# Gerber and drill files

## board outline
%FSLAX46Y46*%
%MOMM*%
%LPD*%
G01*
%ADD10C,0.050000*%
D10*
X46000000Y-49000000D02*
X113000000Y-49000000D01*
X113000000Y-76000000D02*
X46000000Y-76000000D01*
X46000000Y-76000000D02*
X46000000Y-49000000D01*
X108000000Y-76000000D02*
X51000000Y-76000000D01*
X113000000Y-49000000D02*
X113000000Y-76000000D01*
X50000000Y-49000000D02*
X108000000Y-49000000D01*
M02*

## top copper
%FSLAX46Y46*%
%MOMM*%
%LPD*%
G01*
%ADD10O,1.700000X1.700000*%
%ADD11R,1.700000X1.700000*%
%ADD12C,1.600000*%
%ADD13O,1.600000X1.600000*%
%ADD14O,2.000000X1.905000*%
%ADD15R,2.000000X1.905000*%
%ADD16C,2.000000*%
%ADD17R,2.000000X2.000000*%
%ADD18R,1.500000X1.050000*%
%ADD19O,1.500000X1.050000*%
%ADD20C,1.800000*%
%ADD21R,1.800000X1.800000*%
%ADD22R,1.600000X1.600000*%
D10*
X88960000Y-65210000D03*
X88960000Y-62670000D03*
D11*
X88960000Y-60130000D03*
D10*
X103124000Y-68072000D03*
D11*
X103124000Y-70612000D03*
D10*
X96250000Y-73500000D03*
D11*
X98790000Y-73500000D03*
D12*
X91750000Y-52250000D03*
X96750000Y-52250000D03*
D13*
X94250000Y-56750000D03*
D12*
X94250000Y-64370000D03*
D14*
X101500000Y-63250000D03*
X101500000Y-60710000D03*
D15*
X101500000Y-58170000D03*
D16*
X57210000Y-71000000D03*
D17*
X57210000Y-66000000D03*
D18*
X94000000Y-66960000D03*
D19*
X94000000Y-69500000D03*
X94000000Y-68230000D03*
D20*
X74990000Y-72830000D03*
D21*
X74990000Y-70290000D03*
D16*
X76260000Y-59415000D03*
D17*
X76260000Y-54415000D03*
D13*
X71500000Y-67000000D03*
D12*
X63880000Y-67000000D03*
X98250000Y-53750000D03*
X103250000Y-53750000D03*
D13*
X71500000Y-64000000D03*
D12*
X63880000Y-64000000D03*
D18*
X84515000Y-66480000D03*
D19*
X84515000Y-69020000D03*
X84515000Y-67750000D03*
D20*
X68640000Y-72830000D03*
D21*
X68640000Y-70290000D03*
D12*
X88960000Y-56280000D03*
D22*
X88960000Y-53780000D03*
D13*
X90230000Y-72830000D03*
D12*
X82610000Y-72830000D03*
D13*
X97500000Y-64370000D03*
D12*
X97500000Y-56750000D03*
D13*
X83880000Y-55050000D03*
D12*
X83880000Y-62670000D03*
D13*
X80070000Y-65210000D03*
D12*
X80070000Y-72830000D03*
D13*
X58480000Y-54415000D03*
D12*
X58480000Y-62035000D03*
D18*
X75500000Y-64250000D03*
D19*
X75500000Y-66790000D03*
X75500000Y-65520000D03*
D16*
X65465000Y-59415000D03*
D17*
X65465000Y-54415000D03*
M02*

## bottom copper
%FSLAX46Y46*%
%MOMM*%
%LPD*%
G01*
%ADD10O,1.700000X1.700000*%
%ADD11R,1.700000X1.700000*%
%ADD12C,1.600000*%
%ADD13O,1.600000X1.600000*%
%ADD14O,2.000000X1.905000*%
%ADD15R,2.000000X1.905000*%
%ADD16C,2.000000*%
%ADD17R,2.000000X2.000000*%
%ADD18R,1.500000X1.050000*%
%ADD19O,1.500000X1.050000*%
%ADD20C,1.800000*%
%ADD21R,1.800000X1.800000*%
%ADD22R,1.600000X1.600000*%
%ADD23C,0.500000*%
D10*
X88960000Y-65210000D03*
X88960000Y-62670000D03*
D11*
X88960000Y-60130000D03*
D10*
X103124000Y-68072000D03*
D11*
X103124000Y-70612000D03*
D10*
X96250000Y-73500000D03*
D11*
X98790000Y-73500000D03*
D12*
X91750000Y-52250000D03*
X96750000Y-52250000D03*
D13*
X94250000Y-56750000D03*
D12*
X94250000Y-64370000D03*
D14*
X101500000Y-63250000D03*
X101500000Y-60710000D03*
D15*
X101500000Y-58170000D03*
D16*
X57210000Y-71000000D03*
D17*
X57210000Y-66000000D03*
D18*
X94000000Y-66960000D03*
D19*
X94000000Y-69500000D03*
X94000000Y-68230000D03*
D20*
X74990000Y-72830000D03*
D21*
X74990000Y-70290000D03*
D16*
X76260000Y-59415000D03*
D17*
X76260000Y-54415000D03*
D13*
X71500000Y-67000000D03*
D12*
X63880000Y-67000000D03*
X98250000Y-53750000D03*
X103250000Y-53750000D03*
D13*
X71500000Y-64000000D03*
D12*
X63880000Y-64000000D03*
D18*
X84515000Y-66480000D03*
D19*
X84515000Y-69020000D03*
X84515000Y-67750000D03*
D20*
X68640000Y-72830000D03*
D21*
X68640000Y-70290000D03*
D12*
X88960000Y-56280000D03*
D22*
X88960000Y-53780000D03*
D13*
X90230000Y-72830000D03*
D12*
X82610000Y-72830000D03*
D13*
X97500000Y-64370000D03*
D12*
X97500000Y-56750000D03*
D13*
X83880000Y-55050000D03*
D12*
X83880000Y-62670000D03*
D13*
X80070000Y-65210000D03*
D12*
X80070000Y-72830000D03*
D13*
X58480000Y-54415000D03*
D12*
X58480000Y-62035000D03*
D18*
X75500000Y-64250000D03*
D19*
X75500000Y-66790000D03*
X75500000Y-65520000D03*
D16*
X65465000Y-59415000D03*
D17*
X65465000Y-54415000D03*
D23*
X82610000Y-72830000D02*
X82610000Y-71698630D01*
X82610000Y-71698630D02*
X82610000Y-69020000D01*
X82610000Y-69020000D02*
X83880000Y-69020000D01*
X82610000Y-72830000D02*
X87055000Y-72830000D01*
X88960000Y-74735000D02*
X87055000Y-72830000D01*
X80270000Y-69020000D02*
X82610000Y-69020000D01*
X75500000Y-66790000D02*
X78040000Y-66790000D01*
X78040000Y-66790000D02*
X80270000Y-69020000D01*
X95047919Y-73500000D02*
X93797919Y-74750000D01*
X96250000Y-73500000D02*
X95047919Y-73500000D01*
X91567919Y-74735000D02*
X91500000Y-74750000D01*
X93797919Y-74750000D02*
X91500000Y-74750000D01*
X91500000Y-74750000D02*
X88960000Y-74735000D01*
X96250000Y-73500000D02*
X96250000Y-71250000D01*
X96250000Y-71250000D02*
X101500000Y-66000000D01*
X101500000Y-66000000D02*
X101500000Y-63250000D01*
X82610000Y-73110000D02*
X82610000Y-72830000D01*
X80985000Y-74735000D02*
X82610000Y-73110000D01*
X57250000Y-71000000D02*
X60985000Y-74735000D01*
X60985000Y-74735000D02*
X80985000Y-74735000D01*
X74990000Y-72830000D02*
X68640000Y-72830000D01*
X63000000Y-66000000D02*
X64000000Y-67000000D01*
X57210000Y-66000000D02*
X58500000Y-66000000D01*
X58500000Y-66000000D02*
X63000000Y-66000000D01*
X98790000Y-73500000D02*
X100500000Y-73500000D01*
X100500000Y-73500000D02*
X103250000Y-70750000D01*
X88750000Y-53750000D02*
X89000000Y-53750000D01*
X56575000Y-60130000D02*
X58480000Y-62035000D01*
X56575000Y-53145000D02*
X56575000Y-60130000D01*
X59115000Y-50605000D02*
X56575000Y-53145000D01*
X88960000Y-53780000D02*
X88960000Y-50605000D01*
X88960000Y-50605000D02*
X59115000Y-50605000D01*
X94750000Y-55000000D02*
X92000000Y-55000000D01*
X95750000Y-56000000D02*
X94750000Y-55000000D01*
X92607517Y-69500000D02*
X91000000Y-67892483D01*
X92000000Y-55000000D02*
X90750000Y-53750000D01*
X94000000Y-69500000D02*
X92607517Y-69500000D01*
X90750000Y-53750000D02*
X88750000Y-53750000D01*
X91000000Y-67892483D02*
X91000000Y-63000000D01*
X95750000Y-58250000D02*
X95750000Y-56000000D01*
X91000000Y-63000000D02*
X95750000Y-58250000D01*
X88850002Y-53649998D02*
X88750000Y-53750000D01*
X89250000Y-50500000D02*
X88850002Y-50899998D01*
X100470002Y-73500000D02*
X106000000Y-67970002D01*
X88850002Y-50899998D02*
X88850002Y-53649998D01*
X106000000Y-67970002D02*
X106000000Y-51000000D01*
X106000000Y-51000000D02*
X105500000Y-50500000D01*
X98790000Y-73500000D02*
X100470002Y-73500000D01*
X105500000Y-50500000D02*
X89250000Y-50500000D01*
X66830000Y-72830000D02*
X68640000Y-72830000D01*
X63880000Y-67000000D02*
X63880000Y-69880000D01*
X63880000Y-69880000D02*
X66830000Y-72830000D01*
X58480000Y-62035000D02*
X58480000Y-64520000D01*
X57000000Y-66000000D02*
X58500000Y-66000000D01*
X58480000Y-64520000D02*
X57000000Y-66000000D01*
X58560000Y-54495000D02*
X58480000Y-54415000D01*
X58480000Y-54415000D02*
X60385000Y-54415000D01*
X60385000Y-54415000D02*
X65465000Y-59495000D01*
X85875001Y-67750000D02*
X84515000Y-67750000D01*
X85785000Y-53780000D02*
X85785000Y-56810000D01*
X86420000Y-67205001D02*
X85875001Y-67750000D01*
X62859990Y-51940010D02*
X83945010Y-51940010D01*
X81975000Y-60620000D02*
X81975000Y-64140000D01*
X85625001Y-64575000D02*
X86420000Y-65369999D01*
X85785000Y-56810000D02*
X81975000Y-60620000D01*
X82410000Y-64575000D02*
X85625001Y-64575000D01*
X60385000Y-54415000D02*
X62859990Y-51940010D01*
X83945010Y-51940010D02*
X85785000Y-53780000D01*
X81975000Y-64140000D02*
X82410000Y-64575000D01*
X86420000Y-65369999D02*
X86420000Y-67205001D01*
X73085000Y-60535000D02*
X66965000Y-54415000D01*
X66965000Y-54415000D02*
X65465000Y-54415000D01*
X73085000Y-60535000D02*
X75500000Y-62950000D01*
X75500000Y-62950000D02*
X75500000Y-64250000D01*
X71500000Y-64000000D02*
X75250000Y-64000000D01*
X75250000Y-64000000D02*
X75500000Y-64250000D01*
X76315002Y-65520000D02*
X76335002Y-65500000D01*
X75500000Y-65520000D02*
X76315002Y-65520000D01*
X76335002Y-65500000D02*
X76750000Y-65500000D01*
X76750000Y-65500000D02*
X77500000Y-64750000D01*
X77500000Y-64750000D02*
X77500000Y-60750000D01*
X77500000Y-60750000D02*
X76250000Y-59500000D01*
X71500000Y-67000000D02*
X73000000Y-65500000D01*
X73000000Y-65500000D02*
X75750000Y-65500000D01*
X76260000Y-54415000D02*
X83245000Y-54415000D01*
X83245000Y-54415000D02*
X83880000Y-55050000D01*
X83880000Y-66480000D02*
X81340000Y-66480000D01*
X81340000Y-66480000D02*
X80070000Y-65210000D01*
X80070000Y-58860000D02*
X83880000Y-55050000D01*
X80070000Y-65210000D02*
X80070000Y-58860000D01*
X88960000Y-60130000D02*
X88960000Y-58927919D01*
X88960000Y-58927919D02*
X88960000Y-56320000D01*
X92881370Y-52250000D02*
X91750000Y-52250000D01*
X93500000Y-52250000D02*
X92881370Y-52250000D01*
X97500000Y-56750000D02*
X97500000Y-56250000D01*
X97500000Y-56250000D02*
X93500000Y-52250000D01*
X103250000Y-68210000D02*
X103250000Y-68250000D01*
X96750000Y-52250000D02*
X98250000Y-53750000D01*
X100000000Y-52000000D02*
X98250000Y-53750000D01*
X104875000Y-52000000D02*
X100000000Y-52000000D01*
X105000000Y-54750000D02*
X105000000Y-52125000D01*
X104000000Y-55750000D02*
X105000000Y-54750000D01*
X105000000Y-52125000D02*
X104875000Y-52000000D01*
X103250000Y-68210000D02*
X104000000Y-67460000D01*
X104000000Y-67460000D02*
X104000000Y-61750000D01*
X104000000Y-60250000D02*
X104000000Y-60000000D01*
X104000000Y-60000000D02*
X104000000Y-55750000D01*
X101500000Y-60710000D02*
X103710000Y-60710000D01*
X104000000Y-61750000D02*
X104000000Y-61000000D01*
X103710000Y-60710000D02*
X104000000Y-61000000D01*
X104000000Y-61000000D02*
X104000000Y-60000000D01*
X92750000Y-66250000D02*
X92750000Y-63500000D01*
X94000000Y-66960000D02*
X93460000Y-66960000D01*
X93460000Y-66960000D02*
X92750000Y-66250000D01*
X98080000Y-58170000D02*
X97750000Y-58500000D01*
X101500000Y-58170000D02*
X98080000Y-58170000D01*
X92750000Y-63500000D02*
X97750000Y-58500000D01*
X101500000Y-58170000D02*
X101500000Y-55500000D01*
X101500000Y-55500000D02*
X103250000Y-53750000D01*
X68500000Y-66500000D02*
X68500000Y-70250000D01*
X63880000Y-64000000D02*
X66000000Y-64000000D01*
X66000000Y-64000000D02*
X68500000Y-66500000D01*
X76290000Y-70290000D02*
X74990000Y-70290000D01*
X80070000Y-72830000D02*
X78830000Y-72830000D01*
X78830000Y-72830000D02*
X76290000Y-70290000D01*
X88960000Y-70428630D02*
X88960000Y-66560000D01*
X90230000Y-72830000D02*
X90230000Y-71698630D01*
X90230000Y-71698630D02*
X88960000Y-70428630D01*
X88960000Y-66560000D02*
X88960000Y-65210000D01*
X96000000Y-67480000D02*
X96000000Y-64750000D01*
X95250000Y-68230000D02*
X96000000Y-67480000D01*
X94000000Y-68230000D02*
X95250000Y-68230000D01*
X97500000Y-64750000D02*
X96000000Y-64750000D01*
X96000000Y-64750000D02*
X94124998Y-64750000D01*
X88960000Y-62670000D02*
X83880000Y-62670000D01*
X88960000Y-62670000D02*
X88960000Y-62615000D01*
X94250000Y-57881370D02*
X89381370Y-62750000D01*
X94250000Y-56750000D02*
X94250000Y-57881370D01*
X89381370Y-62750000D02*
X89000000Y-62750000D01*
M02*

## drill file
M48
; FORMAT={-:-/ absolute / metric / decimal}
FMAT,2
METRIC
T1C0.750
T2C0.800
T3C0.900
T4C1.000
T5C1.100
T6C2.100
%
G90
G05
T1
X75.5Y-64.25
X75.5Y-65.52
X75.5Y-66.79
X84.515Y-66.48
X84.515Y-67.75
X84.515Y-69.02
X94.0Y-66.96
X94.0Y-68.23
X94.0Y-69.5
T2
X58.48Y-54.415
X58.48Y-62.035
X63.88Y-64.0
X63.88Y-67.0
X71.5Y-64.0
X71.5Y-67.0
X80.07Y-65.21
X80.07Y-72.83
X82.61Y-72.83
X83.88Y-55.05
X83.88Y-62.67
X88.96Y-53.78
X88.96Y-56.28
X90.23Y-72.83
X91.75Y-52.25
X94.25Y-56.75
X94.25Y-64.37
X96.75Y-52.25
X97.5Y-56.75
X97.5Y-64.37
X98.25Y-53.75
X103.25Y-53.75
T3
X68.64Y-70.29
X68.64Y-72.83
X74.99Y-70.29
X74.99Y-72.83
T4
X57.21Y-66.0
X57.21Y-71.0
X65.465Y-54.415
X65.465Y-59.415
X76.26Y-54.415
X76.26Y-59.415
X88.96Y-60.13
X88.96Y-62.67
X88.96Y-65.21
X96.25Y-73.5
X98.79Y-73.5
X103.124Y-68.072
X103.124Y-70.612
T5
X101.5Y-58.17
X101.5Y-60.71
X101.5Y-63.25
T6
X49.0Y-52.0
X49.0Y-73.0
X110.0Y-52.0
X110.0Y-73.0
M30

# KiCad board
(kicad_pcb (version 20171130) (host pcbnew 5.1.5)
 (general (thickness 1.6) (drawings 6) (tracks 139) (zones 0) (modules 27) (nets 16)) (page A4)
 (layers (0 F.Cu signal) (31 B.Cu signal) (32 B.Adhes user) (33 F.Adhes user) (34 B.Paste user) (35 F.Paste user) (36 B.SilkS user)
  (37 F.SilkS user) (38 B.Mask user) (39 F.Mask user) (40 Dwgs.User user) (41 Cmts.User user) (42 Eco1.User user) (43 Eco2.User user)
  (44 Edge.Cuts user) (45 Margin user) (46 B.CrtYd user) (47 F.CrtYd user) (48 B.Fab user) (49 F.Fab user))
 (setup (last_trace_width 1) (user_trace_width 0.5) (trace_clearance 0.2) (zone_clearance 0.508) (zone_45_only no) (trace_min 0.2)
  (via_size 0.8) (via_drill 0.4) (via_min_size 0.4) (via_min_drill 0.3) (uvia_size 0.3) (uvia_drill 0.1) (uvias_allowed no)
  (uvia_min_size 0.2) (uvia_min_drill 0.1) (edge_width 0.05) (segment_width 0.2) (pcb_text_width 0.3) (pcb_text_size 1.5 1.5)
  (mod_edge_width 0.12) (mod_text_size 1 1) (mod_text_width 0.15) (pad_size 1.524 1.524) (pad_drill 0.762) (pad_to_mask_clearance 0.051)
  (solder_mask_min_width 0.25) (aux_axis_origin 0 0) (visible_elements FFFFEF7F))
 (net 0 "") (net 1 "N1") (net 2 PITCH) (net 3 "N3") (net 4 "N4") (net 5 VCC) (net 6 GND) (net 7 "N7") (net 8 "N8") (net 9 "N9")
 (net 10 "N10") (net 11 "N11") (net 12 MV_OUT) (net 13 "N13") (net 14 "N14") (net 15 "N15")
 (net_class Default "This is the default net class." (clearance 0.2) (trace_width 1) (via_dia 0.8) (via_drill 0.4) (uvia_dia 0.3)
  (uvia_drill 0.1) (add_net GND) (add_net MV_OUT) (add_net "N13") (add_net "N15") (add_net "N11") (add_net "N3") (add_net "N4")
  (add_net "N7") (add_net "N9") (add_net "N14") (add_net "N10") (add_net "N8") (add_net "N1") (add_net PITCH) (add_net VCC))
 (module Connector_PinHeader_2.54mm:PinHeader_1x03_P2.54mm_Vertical (layer F.Cu) (at 88.96 60.13)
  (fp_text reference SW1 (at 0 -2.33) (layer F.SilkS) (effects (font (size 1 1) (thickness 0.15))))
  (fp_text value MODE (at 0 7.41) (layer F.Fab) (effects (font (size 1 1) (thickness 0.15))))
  (pad 3 thru_hole oval (at 0 5.08) (size 1.7 1.7) (drill 1) (layers *.Cu *.Mask) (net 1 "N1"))
  (pad 2 thru_hole oval (at 0 2.54) (size 1.7 1.7) (drill 1) (layers *.Cu *.Mask) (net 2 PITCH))
  (pad 1 thru_hole rect (at 0 0) (size 1.7 1.7) (drill 1) (layers *.Cu *.Mask) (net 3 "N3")))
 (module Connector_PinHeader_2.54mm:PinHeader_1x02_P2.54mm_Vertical (layer F.Cu) (at 103.124 70.612 180)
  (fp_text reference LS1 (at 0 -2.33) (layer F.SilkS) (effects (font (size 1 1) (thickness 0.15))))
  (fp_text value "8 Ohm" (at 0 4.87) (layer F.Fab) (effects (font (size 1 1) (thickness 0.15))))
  (pad 2 thru_hole oval (at 0 2.54 180) (size 1.7 1.7) (drill 1) (layers *.Cu *.Mask) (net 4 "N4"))
  (pad 1 thru_hole rect (at 0 0 180) (size 1.7 1.7) (drill 1) (layers *.Cu *.Mask) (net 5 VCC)))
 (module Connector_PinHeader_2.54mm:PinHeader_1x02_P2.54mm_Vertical (layer F.Cu) (at 98.79 73.5 270)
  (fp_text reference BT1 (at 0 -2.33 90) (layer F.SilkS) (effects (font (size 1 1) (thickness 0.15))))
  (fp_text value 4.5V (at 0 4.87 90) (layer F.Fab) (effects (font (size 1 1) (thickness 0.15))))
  (pad 2 thru_hole oval (at 0 2.54 270) (size 1.7 1.7) (drill 1) (layers *.Cu *.Mask) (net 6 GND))
  (pad 1 thru_hole rect (at 0 0 270) (size 1.7 1.7) (drill 1) (layers *.Cu *.Mask) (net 5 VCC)))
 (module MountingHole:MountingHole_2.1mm (layer F.Cu) (at 110 73)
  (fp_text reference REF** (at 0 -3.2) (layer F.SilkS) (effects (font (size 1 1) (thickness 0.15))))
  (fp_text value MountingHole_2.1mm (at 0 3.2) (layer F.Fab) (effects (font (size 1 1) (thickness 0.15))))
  (pad "" np_thru_hole circle (at 0 0) (size 2.1 2.1) (drill 2.1) (layers *.Cu *.Mask)))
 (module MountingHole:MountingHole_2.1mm (layer F.Cu) (at 110 52)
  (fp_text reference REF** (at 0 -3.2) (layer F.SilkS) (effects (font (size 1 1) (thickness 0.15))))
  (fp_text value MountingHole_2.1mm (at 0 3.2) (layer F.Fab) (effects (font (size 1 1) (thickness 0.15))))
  (pad "" np_thru_hole circle (at 0 0) (size 2.1 2.1) (drill 2.1) (layers *.Cu *.Mask)))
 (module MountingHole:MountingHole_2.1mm (layer F.Cu) (at 49 73)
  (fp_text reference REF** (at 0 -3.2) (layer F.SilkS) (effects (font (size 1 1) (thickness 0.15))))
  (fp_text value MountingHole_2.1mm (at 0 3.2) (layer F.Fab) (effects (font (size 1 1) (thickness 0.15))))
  (pad "" np_thru_hole circle (at 0 0) (size 2.1 2.1) (drill 2.1) (layers *.Cu *.Mask)))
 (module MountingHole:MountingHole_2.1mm (layer F.Cu) (at 49 52)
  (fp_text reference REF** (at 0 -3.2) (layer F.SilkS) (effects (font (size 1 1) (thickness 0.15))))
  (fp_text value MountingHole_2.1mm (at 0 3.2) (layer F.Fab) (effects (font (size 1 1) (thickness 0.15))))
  (pad "" np_thru_hole circle (at 0 0) (size 2.1 2.1) (drill 2.1) (layers *.Cu *.Mask)))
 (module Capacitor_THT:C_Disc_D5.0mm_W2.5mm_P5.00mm (layer F.Cu) (at 96.75 52.25 180)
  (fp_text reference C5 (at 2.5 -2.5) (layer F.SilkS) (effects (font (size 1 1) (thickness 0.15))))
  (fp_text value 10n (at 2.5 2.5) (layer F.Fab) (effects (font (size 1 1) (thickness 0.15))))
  (pad 2 thru_hole circle (at 5 0 180) (size 1.6 1.6) (drill 0.8) (layers *.Cu *.Mask) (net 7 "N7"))
  (pad 1 thru_hole circle (at 0 0 180) (size 1.6 1.6) (drill 0.8) (layers *.Cu *.Mask) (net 4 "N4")))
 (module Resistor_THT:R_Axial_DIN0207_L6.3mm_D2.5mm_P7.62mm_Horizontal (layer F.Cu) (at 94.25 64.37 90)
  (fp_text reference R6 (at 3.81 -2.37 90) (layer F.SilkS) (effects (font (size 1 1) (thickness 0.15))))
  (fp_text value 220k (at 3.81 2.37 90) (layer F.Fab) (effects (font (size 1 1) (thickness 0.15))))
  (pad 2 thru_hole oval (at 7.62 0 90) (size 1.6 1.6) (drill 0.8) (layers *.Cu *.Mask) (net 2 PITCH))
  (pad 1 thru_hole circle (at 0 0 90) (size 1.6 1.6) (drill 0.8) (layers *.Cu *.Mask) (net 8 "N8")))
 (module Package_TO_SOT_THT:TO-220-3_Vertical (layer F.Cu) (at 101.5 58.17 270)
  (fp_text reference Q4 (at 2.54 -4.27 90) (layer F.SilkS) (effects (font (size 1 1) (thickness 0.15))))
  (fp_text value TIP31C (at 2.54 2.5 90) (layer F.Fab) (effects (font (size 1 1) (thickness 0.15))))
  (pad 3 thru_hole oval (at 5.08 0 270) (size 1.905 2) (drill 1.1) (layers *.Cu *.Mask) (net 6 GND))
  (pad 2 thru_hole oval (at 2.54 0 270) (size 1.905 2) (drill 1.1) (layers *.Cu *.Mask) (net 4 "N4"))
  (pad 1 thru_hole rect (at 0 0 270) (size 1.905 2) (drill 1.1) (layers *.Cu *.Mask) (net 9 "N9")))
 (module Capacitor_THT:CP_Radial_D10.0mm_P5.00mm (layer F.Cu) (at 57.21 66 270)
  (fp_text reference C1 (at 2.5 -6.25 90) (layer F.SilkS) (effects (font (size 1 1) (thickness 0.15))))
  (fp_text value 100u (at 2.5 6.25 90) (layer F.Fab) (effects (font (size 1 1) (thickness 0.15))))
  (pad 2 thru_hole circle (at 5 0 270) (size 2 2) (drill 1) (layers *.Cu *.Mask) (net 6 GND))
  (pad 1 thru_hole rect (at 0 0 270) (size 2 2) (drill 1) (layers *.Cu *.Mask) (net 5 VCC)))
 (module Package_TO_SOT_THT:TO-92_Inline (layer F.Cu) (at 94 66.96 270)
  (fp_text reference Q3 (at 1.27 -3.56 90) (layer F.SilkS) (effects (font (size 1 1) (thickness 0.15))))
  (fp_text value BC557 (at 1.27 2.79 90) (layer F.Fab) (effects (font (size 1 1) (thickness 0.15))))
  (pad 1 thru_hole rect (at 0 0 270) (size 1.05 1.5) (drill 0.75) (layers *.Cu *.Mask) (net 9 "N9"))
  (pad 3 thru_hole oval (at 2.54 0 270) (size 1.05 1.5) (drill 0.75) (layers *.Cu *.Mask) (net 5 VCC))
  (pad 2 thru_hole oval (at 1.27 0 270) (size 1.05 1.5) (drill 0.75) (layers *.Cu *.Mask) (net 8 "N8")))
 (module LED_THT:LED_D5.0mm (layer F.Cu) (at 74.99 70.29 270)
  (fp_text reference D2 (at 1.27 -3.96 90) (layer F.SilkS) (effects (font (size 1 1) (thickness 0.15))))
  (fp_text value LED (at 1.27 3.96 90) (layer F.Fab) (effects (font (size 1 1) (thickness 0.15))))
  (pad 2 thru_hole circle (at 2.54 0 270) (size 1.8 1.8) (drill 0.9) (layers *.Cu *.Mask) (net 5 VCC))
  (pad 1 thru_hole rect (at 0 0 270) (size 1.8 1.8) (drill 0.9) (layers *.Cu *.Mask) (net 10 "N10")))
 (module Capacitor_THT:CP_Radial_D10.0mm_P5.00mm (layer F.Cu) (at 76.26 54.415 270)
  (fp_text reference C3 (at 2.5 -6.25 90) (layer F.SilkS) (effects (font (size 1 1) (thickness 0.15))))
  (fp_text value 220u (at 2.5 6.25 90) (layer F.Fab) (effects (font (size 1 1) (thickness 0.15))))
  (pad 2 thru_hole circle (at 5 0 270) (size 2 2) (drill 1) (layers *.Cu *.Mask) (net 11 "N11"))
  (pad 1 thru_hole rect (at 0 0 270) (size 2 2) (drill 1) (layers *.Cu *.Mask) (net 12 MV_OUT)))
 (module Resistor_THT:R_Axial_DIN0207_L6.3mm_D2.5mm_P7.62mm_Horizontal (layer F.Cu) (at 63.88 67)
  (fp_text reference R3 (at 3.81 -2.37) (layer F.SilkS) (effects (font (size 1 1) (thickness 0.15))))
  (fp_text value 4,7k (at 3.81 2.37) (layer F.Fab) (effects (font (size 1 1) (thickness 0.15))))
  (pad 2 thru_hole oval (at 7.62 0) (size 1.6 1.6) (drill 0.8) (layers *.Cu *.Mask) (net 11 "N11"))
  (pad 1 thru_hole circle (at 0 0) (size 1.6 1.6) (drill 0.8) (layers *.Cu *.Mask) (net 5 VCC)))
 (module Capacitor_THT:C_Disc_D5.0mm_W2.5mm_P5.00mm (layer F.Cu) (at 103.25 53.75 180)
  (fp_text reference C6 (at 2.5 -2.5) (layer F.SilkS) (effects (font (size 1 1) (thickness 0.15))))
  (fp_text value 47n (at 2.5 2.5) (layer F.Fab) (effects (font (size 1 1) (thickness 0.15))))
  (pad 2 thru_hole circle (at 5 0 180) (size 1.6 1.6) (drill 0.8) (layers *.Cu *.Mask) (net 4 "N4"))
  (pad 1 thru_hole circle (at 0 0 180) (size 1.6 1.6) (drill 0.8) (layers *.Cu *.Mask) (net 9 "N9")))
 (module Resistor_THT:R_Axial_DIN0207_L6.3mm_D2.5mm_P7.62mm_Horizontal (layer F.Cu) (at 63.88 64)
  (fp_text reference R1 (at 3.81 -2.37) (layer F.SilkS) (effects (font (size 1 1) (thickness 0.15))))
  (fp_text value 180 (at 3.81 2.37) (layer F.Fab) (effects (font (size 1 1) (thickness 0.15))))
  (pad 2 thru_hole oval (at 7.62 0) (size 1.6 1.6) (drill 0.8) (layers *.Cu *.Mask) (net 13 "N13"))
  (pad 1 thru_hole circle (at 0 0) (size 1.6 1.6) (drill 0.8) (layers *.Cu *.Mask) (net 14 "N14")))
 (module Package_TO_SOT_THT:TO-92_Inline (layer F.Cu) (at 84.515 66.48 270)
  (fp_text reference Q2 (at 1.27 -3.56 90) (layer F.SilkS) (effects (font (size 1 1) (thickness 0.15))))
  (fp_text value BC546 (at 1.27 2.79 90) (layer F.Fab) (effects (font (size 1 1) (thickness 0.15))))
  (pad 1 thru_hole rect (at 0 0 270) (size 1.05 1.5) (drill 0.75) (layers *.Cu *.Mask) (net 12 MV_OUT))
  (pad 3 thru_hole oval (at 2.54 0 270) (size 1.05 1.5) (drill 0.75) (layers *.Cu *.Mask) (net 6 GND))
  (pad 2 thru_hole oval (at 1.27 0 270) (size 1.05 1.5) (drill 0.75) (layers *.Cu *.Mask) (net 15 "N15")))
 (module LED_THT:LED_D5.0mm (layer F.Cu) (at 68.64 70.29 270)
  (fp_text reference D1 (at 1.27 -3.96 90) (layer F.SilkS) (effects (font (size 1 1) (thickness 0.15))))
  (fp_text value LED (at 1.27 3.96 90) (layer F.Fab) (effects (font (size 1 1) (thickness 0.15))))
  (pad 2 thru_hole circle (at 2.54 0 270) (size 1.8 1.8) (drill 0.9) (layers *.Cu *.Mask) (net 5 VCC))
  (pad 1 thru_hole rect (at 0 0 270) (size 1.8 1.8) (drill 0.9) (layers *.Cu *.Mask) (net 14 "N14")))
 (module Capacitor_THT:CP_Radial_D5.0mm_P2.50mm (layer F.Cu) (at 88.96 53.78 270)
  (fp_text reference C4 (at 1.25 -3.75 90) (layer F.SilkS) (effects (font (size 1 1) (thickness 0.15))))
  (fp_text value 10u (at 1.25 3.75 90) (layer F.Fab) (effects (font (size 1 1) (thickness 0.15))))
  (pad 2 thru_hole circle (at 2.5 0 270) (size 1.6 1.6) (drill 0.8) (layers *.Cu *.Mask) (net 3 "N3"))
  (pad 1 thru_hole rect (at 0 0 270) (size 1.6 1.6) (drill 0.8) (layers *.Cu *.Mask) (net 5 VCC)))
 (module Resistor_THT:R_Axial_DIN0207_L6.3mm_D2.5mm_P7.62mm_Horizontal (layer F.Cu) (at 82.61 72.83)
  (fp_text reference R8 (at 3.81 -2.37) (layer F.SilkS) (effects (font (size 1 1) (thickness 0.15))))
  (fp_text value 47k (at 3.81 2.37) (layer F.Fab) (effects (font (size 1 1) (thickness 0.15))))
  (pad 2 thru_hole oval (at 7.62 0) (size 1.6 1.6) (drill 0.8) (layers *.Cu *.Mask) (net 1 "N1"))
  (pad 1 thru_hole circle (at 0 0) (size 1.6 1.6) (drill 0.8) (layers *.Cu *.Mask) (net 6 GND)))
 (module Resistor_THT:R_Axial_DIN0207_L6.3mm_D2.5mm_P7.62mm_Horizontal (layer F.Cu) (at 97.5 56.75 270)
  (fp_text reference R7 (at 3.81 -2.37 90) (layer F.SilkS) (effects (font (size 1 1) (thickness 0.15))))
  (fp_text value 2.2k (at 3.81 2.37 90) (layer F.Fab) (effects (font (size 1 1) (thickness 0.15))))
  (pad 2 thru_hole oval (at 7.62 0 270) (size 1.6 1.6) (drill 0.8) (layers *.Cu *.Mask) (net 8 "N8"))
  (pad 1 thru_hole circle (at 0 0 270) (size 1.6 1.6) (drill 0.8) (layers *.Cu *.Mask) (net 7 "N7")))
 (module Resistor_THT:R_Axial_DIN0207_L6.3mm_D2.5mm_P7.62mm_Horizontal (layer F.Cu) (at 83.88 62.67 90)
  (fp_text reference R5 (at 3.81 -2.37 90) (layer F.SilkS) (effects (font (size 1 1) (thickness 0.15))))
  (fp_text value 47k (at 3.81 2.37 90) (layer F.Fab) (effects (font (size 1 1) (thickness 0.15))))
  (pad 2 thru_hole oval (at 7.62 0 90) (size 1.6 1.6) (drill 0.8) (layers *.Cu *.Mask) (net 12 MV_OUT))
  (pad 1 thru_hole circle (at 0 0 90) (size 1.6 1.6) (drill 0.8) (layers *.Cu *.Mask) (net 2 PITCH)))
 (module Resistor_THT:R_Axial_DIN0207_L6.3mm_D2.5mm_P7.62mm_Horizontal (layer F.Cu) (at 80.07 72.83 90)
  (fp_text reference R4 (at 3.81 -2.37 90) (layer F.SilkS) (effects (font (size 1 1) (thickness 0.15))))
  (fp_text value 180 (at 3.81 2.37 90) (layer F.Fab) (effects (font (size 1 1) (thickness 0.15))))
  (pad 2 thru_hole oval (at 7.62 0 90) (size 1.6 1.6) (drill 0.8) (layers *.Cu *.Mask) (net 12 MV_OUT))
  (pad 1 thru_hole circle (at 0 0 90) (size 1.6 1.6) (drill 0.8) (layers *.Cu *.Mask) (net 10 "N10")))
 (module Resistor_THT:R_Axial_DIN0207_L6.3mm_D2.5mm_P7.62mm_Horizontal (layer F.Cu) (at 58.48 62.035 90)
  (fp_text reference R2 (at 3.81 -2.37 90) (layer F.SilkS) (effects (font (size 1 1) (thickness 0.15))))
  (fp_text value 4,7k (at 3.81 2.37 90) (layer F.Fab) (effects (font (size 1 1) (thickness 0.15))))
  (pad 2 thru_hole oval (at 7.62 0 90) (size 1.6 1.6) (drill 0.8) (layers *.Cu *.Mask) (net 15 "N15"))
  (pad 1 thru_hole circle (at 0 0 90) (size 1.6 1.6) (drill 0.8) (layers *.Cu *.Mask) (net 5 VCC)))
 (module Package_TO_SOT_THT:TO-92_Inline (layer F.Cu) (at 75.5 64.25 270)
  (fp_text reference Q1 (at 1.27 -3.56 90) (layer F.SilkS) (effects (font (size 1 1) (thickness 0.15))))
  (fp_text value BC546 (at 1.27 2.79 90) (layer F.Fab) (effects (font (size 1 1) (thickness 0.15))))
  (pad 1 thru_hole rect (at 0 0 270) (size 1.05 1.5) (drill 0.75) (layers *.Cu *.Mask) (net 13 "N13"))
  (pad 3 thru_hole oval (at 2.54 0 270) (size 1.05 1.5) (drill 0.75) (layers *.Cu *.Mask) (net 6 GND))
  (pad 2 thru_hole oval (at 1.27 0 270) (size 1.05 1.5) (drill 0.75) (layers *.Cu *.Mask) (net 11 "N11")))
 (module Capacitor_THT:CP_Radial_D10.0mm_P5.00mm (layer F.Cu) (at 65.465 54.415 270)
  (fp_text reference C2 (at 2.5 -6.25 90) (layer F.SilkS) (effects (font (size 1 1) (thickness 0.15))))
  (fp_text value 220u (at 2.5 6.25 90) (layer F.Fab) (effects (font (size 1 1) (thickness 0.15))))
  (pad 2 thru_hole circle (at 5 0 270) (size 2 2) (drill 1) (layers *.Cu *.Mask) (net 15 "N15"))
  (pad 1 thru_hole rect (at 0 0 270) (size 2 2) (drill 1) (layers *.Cu *.Mask) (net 13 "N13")))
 (gr_line (start 46 49) (end 113 49) (layer Edge.Cuts) (width 0.05))
 (gr_line (start 113 76) (end 46 76) (layer Edge.Cuts) (width 0.05))
 (gr_line (start 46 76) (end 46 49) (layer Edge.Cuts) (width 0.05))
 (gr_line (start 108 76) (end 51 76) (layer Edge.Cuts) (width 0.05))
 (gr_line (start 113 49) (end 113 76) (layer Edge.Cuts) (width 0.05))
 (gr_line (start 50 49) (end 108 49) (layer Edge.Cuts) (width 0.05))
 (segment (start 82.61 72.83) (end 82.61 71.69863) (width 0.5) (layer B.Cu) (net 6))
 (segment (start 82.61 71.69863) (end 82.61 69.02) (width 0.5) (layer B.Cu) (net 6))
 (segment (start 82.61 69.02) (end 83.88 69.02) (width 0.5) (layer B.Cu) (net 6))
 (segment (start 82.61 72.83) (end 87.055 72.83) (width 0.5) (layer B.Cu) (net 6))
 (segment (start 88.96 74.735) (end 87.055 72.83) (width 0.5) (layer B.Cu) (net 6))
 (segment (start 80.27 69.02) (end 82.61 69.02) (width 0.5) (layer B.Cu) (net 6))
 (segment (start 75.5 66.79) (end 78.04 66.79) (width 0.5) (layer B.Cu) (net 6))
 (segment (start 78.04 66.79) (end 80.27 69.02) (width 0.5) (layer B.Cu) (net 6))
 (segment (start 95.047919 73.5) (end 93.797919 74.75) (width 0.5) (layer B.Cu) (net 6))
 (segment (start 96.25 73.5) (end 95.047919 73.5) (width 0.5) (layer B.Cu) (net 6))
 (segment (start 91.567919 74.735) (end 91.5 74.75) (width 0.5) (layer B.Cu) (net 6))
 (segment (start 93.797919 74.75) (end 91.5 74.75) (width 0.5) (layer B.Cu) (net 6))
 (segment (start 91.5 74.75) (end 88.96 74.735) (width 0.5) (layer B.Cu) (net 6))
 (segment (start 96.25 73.5) (end 96.25 71.25) (width 0.5) (layer B.Cu) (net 6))
 (segment (start 96.25 71.25) (end 101.5 66) (width 0.5) (layer B.Cu) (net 6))
 (segment (start 101.5 66) (end 101.5 63.25) (width 0.5) (layer B.Cu) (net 6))
 (segment (start 82.61 73.11) (end 82.61 72.83) (width 0.5) (layer B.Cu) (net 6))
 (segment (start 80.985 74.735) (end 82.61 73.11) (width 0.5) (layer B.Cu) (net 6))
 (segment (start 57.25 71) (end 60.985 74.735) (width 0.5) (layer B.Cu) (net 6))
 (segment (start 60.985 74.735) (end 80.985 74.735) (width 0.5) (layer B.Cu) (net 6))
 (segment (start 74.99 72.83) (end 68.64 72.83) (width 0.5) (layer B.Cu) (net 5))
 (segment (start 63 66) (end 64 67) (width 0.5) (layer B.Cu) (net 5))
 (segment (start 57.21 66) (end 58.5 66) (width 0.5) (layer B.Cu) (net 5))
 (segment (start 58.5 66) (end 63 66) (width 0.5) (layer B.Cu) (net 5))
 (segment (start 98.79 73.5) (end 100.5 73.5) (width 0.5) (layer B.Cu) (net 5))
 (segment (start 100.5 73.5) (end 103.25 70.75) (width 0.5) (layer B.Cu) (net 5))
 (segment (start 88.75 53.75) (end 89 53.75) (width 0.5) (layer B.Cu) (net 5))
 (segment (start 56.575 60.13) (end 58.48 62.035) (width 0.5) (layer B.Cu) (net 5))
 (segment (start 56.575 53.145) (end 56.575 60.13) (width 0.5) (layer B.Cu) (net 5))
 (segment (start 59.115 50.605) (end 56.575 53.145) (width 0.5) (layer B.Cu) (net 5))
 (segment (start 88.96 53.78) (end 88.96 50.605) (width 0.5) (layer B.Cu) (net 5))
 (segment (start 88.96 50.605) (end 59.115 50.605) (width 0.5) (layer B.Cu) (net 5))
 (segment (start 94.75 55) (end 92 55) (width 0.5) (layer B.Cu) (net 5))
 (segment (start 95.75 56) (end 94.75 55) (width 0.5) (layer B.Cu) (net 5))
 (segment (start 92.607517 69.5) (end 91 67.892483) (width 0.5) (layer B.Cu) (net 5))
 (segment (start 92 55) (end 90.75 53.75) (width 0.5) (layer B.Cu) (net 5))
 (segment (start 94 69.5) (end 92.607517 69.5) (width 0.5) (layer B.Cu) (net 5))
 (segment (start 90.75 53.75) (end 88.75 53.75) (width 0.5) (layer B.Cu) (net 5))
 (segment (start 91 67.892483) (end 91 63) (width 0.5) (layer B.Cu) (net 5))
 (segment (start 95.75 58.25) (end 95.75 56) (width 0.5) (layer B.Cu) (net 5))
 (segment (start 91 63) (end 95.75 58.25) (width 0.5) (layer B.Cu) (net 5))
 (segment (start 88.850002 53.649998) (end 88.75 53.75) (width 0.5) (layer B.Cu) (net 5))
 (segment (start 89.25 50.5) (end 88.850002 50.899998) (width 0.5) (layer B.Cu) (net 5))
 (segment (start 100.470002 73.5) (end 106 67.970002) (width 0.5) (layer B.Cu) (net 5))
 (segment (start 88.850002 50.899998) (end 88.850002 53.649998) (width 0.5) (layer B.Cu) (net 5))
 (segment (start 106 67.970002) (end 106 51) (width 0.5) (layer B.Cu) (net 5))
 (segment (start 106 51) (end 105.5 50.5) (width 0.5) (layer B.Cu) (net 5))
 (segment (start 98.79 73.5) (end 100.470002 73.5) (width 0.5) (layer B.Cu) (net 5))
 (segment (start 105.5 50.5) (end 89.25 50.5) (width 0.5) (layer B.Cu) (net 5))
 (segment (start 66.83 72.83) (end 68.64 72.83) (width 0.5) (layer B.Cu) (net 5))
 (segment (start 63.88 67) (end 63.88 69.88) (width 0.5) (layer B.Cu) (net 5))
 (segment (start 63.88 69.88) (end 66.83 72.83) (width 0.5) (layer B.Cu) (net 5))
 (segment (start 58.48 62.035) (end 58.48 64.52) (width 0.5) (layer B.Cu) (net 5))
 (segment (start 57 66) (end 58.5 66) (width 0.5) (layer B.Cu) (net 5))
 (segment (start 58.48 64.52) (end 57 66) (width 0.5) (layer B.Cu) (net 5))
 (segment (start 58.56 54.495) (end 58.48 54.415) (width 0.5) (layer B.Cu) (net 15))
 (segment (start 58.48 54.415) (end 60.385 54.415) (width 0.5) (layer B.Cu) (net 15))
 (segment (start 60.385 54.415) (end 65.465 59.495) (width 0.5) (layer B.Cu) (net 15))
 (segment (start 85.875001 67.75) (end 84.515 67.75) (width 0.5) (layer B.Cu) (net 15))
 (segment (start 85.785 53.78) (end 85.785 56.81) (width 0.5) (layer B.Cu) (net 15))
 (segment (start 86.42 67.205001) (end 85.875001 67.75) (width 0.5) (layer B.Cu) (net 15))
 (segment (start 62.85999 51.94001) (end 83.94501 51.94001) (width 0.5) (layer B.Cu) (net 15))
 (segment (start 81.975 60.62) (end 81.975 64.14) (width 0.5) (layer B.Cu) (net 15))
 (segment (start 85.625001 64.575) (end 86.42 65.369999) (width 0.5) (layer B.Cu) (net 15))
 (segment (start 85.785 56.81) (end 81.975 60.62) (width 0.5) (layer B.Cu) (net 15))
 (segment (start 82.41 64.575) (end 85.625001 64.575) (width 0.5) (layer B.Cu) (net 15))
 (segment (start 60.385 54.415) (end 62.85999 51.94001) (width 0.5) (layer B.Cu) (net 15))
 (segment (start 83.94501 51.94001) (end 85.785 53.78) (width 0.5) (layer B.Cu) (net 15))
 (segment (start 81.975 64.14) (end 82.41 64.575) (width 0.5) (layer B.Cu) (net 15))
 (segment (start 86.42 65.369999) (end 86.42 67.205001) (width 0.5) (layer B.Cu) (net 15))
 (segment (start 73.085 60.535) (end 66.965 54.415) (width 0.5) (layer B.Cu) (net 13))
 (segment (start 66.965 54.415) (end 65.465 54.415) (width 0.5) (layer B.Cu) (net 13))
 (segment (start 73.085 60.535) (end 75.5 62.95) (width 0.5) (layer B.Cu) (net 13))
 (segment (start 75.5 62.95) (end 75.5 64.25) (width 0.5) (layer B.Cu) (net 13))
 (segment (start 71.5 64) (end 75.25 64) (width 0.5) (layer B.Cu) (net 13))
 (segment (start 75.25 64) (end 75.5 64.25) (width 0.5) (layer B.Cu) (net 13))
 (segment (start 76.315002 65.52) (end 76.335002 65.5) (width 0.5) (layer B.Cu) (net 11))
 (segment (start 75.5 65.52) (end 76.315002 65.52) (width 0.5) (layer B.Cu) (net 11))
 (segment (start 76.335002 65.5) (end 76.75 65.5) (width 0.5) (layer B.Cu) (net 11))
 (segment (start 76.75 65.5) (end 77.5 64.75) (width 0.5) (layer B.Cu) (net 11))
 (segment (start 77.5 64.75) (end 77.5 60.75) (width 0.5) (layer B.Cu) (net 11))
 (segment (start 77.5 60.75) (end 76.25 59.5) (width 0.5) (layer B.Cu) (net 11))
 (segment (start 71.5 67) (end 73 65.5) (width 0.5) (layer B.Cu) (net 11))
 (segment (start 73 65.5) (end 75.75 65.5) (width 0.5) (layer B.Cu) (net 11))
 (segment (start 76.26 54.415) (end 83.245 54.415) (width 0.5) (layer B.Cu) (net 12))
 (segment (start 83.245 54.415) (end 83.88 55.05) (width 0.5) (layer B.Cu) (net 12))
 (segment (start 83.88 66.48) (end 81.34 66.48) (width 0.5) (layer B.Cu) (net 12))
 (segment (start 81.34 66.48) (end 80.07 65.21) (width 0.5) (layer B.Cu) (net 12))
 (segment (start 80.07 58.86) (end 83.88 55.05) (width 0.5) (layer B.Cu) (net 12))
 (segment (start 80.07 65.21) (end 80.07 58.86) (width 0.5) (layer B.Cu) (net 12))
 (segment (start 88.96 60.13) (end 88.96 58.927919) (width 0.5) (layer B.Cu) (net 3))
 (segment (start 88.96 58.927919) (end 88.96 56.32) (width 0.5) (layer B.Cu) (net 3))
 (segment (start 92.88137 52.25) (end 91.75 52.25) (width 0.5) (layer B.Cu) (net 7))
 (segment (start 93.5 52.25) (end 92.88137 52.25) (width 0.5) (layer B.Cu) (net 7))
 (segment (start 97.5 56.75) (end 97.5 56.25) (width 0.5) (layer B.Cu) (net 7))
 (segment (start 97.5 56.25) (end 93.5 52.25) (width 0.5) (layer B.Cu) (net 7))
 (segment (start 103.25 68.21) (end 103.25 68.25) (width 0.5) (layer B.Cu) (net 4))
 (segment (start 96.75 52.25) (end 98.25 53.75) (width 0.5) (layer B.Cu) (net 4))
 (segment (start 100 52) (end 98.25 53.75) (width 0.5) (layer B.Cu) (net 4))
 (segment (start 104.875 52) (end 100 52) (width 0.5) (layer B.Cu) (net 4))
 (segment (start 105 54.75) (end 105 52.125) (width 0.5) (layer B.Cu) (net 4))
 (segment (start 104 55.75) (end 105 54.75) (width 0.5) (layer B.Cu) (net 4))
 (segment (start 105 52.125) (end 104.875 52) (width 0.5) (layer B.Cu) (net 4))
 (segment (start 103.25 68.21) (end 104 67.46) (width 0.5) (layer B.Cu) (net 4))
 (segment (start 104 67.46) (end 104 61.75) (width 0.5) (layer B.Cu) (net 4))
 (segment (start 104 60.25) (end 104 60) (width 0.5) (layer B.Cu) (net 4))
 (segment (start 104 60) (end 104 55.75) (width 0.5) (layer B.Cu) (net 4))
 (segment (start 101.5 60.71) (end 103.71 60.71) (width 0.5) (layer B.Cu) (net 4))
 (segment (start 104 61.75) (end 104 61) (width 0.5) (layer B.Cu) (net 4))
 (segment (start 103.71 60.71) (end 104 61) (width 0.5) (layer B.Cu) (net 4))
 (segment (start 104 61) (end 104 60) (width 0.5) (layer B.Cu) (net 4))
 (segment (start 92.75 66.25) (end 92.75 63.5) (width 0.5) (layer B.Cu) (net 9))
 (segment (start 94 66.96) (end 93.46 66.96) (width 0.5) (layer B.Cu) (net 9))
 (segment (start 93.46 66.96) (end 92.75 66.25) (width 0.5) (layer B.Cu) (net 9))
 (segment (start 98.08 58.17) (end 97.75 58.5) (width 0.5) (layer B.Cu) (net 9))
 (segment (start 101.5 58.17) (end 98.08 58.17) (width 0.5) (layer B.Cu) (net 9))
 (segment (start 92.75 63.5) (end 97.75 58.5) (width 0.5) (layer B.Cu) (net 9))
 (segment (start 101.5 58.17) (end 101.5 55.5) (width 0.5) (layer B.Cu) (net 9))
 (segment (start 101.5 55.5) (end 103.25 53.75) (width 0.5) (layer B.Cu) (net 9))
 (segment (start 68.5 66.5) (end 68.5 70.25) (width 0.5) (layer B.Cu) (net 14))
 (segment (start 63.88 64) (end 66 64) (width 0.5) (layer B.Cu) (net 14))
 (segment (start 66 64) (end 68.5 66.5) (width 0.5) (layer B.Cu) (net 14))
 (segment (start 76.29 70.29) (end 74.99 70.29) (width 0.5) (layer B.Cu) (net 10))
 (segment (start 80.07 72.83) (end 78.83 72.83) (width 0.5) (layer B.Cu) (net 10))
 (segment (start 78.83 72.83) (end 76.29 70.29) (width 0.5) (layer B.Cu) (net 10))
 (segment (start 88.96 70.42863) (end 88.96 66.56) (width 0.5) (layer B.Cu) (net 1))
 (segment (start 90.23 72.83) (end 90.23 71.69863) (width 0.5) (layer B.Cu) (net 1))
 (segment (start 90.23 71.69863) (end 88.96 70.42863) (width 0.5) (layer B.Cu) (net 1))
 (segment (start 88.96 66.56) (end 88.96 65.21) (width 0.5) (layer B.Cu) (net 1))
 (segment (start 96 67.48) (end 96 64.75) (width 0.5) (layer B.Cu) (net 8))
 (segment (start 95.25 68.23) (end 96 67.48) (width 0.5) (layer B.Cu) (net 8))
 (segment (start 94 68.23) (end 95.25 68.23) (width 0.5) (layer B.Cu) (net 8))
 (segment (start 97.5 64.75) (end 96 64.75) (width 0.5) (layer B.Cu) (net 8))
 (segment (start 96 64.75) (end 94.124998 64.75) (width 0.5) (layer B.Cu) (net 8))
 (segment (start 88.96 62.67) (end 83.88 62.67) (width 0.5) (layer B.Cu) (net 2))
 (segment (start 88.96 62.67) (end 88.96 62.615) (width 0.5) (layer B.Cu) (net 2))
 (segment (start 94.25 57.88137) (end 89.38137 62.75) (width 0.5) (layer B.Cu) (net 2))
 (segment (start 94.25 56.75) (end 94.25 57.88137) (width 0.5) (layer B.Cu) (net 2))
 (segment (start 89.38137 62.75) (end 89 62.75) (width 0.5) (layer B.Cu) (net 2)))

